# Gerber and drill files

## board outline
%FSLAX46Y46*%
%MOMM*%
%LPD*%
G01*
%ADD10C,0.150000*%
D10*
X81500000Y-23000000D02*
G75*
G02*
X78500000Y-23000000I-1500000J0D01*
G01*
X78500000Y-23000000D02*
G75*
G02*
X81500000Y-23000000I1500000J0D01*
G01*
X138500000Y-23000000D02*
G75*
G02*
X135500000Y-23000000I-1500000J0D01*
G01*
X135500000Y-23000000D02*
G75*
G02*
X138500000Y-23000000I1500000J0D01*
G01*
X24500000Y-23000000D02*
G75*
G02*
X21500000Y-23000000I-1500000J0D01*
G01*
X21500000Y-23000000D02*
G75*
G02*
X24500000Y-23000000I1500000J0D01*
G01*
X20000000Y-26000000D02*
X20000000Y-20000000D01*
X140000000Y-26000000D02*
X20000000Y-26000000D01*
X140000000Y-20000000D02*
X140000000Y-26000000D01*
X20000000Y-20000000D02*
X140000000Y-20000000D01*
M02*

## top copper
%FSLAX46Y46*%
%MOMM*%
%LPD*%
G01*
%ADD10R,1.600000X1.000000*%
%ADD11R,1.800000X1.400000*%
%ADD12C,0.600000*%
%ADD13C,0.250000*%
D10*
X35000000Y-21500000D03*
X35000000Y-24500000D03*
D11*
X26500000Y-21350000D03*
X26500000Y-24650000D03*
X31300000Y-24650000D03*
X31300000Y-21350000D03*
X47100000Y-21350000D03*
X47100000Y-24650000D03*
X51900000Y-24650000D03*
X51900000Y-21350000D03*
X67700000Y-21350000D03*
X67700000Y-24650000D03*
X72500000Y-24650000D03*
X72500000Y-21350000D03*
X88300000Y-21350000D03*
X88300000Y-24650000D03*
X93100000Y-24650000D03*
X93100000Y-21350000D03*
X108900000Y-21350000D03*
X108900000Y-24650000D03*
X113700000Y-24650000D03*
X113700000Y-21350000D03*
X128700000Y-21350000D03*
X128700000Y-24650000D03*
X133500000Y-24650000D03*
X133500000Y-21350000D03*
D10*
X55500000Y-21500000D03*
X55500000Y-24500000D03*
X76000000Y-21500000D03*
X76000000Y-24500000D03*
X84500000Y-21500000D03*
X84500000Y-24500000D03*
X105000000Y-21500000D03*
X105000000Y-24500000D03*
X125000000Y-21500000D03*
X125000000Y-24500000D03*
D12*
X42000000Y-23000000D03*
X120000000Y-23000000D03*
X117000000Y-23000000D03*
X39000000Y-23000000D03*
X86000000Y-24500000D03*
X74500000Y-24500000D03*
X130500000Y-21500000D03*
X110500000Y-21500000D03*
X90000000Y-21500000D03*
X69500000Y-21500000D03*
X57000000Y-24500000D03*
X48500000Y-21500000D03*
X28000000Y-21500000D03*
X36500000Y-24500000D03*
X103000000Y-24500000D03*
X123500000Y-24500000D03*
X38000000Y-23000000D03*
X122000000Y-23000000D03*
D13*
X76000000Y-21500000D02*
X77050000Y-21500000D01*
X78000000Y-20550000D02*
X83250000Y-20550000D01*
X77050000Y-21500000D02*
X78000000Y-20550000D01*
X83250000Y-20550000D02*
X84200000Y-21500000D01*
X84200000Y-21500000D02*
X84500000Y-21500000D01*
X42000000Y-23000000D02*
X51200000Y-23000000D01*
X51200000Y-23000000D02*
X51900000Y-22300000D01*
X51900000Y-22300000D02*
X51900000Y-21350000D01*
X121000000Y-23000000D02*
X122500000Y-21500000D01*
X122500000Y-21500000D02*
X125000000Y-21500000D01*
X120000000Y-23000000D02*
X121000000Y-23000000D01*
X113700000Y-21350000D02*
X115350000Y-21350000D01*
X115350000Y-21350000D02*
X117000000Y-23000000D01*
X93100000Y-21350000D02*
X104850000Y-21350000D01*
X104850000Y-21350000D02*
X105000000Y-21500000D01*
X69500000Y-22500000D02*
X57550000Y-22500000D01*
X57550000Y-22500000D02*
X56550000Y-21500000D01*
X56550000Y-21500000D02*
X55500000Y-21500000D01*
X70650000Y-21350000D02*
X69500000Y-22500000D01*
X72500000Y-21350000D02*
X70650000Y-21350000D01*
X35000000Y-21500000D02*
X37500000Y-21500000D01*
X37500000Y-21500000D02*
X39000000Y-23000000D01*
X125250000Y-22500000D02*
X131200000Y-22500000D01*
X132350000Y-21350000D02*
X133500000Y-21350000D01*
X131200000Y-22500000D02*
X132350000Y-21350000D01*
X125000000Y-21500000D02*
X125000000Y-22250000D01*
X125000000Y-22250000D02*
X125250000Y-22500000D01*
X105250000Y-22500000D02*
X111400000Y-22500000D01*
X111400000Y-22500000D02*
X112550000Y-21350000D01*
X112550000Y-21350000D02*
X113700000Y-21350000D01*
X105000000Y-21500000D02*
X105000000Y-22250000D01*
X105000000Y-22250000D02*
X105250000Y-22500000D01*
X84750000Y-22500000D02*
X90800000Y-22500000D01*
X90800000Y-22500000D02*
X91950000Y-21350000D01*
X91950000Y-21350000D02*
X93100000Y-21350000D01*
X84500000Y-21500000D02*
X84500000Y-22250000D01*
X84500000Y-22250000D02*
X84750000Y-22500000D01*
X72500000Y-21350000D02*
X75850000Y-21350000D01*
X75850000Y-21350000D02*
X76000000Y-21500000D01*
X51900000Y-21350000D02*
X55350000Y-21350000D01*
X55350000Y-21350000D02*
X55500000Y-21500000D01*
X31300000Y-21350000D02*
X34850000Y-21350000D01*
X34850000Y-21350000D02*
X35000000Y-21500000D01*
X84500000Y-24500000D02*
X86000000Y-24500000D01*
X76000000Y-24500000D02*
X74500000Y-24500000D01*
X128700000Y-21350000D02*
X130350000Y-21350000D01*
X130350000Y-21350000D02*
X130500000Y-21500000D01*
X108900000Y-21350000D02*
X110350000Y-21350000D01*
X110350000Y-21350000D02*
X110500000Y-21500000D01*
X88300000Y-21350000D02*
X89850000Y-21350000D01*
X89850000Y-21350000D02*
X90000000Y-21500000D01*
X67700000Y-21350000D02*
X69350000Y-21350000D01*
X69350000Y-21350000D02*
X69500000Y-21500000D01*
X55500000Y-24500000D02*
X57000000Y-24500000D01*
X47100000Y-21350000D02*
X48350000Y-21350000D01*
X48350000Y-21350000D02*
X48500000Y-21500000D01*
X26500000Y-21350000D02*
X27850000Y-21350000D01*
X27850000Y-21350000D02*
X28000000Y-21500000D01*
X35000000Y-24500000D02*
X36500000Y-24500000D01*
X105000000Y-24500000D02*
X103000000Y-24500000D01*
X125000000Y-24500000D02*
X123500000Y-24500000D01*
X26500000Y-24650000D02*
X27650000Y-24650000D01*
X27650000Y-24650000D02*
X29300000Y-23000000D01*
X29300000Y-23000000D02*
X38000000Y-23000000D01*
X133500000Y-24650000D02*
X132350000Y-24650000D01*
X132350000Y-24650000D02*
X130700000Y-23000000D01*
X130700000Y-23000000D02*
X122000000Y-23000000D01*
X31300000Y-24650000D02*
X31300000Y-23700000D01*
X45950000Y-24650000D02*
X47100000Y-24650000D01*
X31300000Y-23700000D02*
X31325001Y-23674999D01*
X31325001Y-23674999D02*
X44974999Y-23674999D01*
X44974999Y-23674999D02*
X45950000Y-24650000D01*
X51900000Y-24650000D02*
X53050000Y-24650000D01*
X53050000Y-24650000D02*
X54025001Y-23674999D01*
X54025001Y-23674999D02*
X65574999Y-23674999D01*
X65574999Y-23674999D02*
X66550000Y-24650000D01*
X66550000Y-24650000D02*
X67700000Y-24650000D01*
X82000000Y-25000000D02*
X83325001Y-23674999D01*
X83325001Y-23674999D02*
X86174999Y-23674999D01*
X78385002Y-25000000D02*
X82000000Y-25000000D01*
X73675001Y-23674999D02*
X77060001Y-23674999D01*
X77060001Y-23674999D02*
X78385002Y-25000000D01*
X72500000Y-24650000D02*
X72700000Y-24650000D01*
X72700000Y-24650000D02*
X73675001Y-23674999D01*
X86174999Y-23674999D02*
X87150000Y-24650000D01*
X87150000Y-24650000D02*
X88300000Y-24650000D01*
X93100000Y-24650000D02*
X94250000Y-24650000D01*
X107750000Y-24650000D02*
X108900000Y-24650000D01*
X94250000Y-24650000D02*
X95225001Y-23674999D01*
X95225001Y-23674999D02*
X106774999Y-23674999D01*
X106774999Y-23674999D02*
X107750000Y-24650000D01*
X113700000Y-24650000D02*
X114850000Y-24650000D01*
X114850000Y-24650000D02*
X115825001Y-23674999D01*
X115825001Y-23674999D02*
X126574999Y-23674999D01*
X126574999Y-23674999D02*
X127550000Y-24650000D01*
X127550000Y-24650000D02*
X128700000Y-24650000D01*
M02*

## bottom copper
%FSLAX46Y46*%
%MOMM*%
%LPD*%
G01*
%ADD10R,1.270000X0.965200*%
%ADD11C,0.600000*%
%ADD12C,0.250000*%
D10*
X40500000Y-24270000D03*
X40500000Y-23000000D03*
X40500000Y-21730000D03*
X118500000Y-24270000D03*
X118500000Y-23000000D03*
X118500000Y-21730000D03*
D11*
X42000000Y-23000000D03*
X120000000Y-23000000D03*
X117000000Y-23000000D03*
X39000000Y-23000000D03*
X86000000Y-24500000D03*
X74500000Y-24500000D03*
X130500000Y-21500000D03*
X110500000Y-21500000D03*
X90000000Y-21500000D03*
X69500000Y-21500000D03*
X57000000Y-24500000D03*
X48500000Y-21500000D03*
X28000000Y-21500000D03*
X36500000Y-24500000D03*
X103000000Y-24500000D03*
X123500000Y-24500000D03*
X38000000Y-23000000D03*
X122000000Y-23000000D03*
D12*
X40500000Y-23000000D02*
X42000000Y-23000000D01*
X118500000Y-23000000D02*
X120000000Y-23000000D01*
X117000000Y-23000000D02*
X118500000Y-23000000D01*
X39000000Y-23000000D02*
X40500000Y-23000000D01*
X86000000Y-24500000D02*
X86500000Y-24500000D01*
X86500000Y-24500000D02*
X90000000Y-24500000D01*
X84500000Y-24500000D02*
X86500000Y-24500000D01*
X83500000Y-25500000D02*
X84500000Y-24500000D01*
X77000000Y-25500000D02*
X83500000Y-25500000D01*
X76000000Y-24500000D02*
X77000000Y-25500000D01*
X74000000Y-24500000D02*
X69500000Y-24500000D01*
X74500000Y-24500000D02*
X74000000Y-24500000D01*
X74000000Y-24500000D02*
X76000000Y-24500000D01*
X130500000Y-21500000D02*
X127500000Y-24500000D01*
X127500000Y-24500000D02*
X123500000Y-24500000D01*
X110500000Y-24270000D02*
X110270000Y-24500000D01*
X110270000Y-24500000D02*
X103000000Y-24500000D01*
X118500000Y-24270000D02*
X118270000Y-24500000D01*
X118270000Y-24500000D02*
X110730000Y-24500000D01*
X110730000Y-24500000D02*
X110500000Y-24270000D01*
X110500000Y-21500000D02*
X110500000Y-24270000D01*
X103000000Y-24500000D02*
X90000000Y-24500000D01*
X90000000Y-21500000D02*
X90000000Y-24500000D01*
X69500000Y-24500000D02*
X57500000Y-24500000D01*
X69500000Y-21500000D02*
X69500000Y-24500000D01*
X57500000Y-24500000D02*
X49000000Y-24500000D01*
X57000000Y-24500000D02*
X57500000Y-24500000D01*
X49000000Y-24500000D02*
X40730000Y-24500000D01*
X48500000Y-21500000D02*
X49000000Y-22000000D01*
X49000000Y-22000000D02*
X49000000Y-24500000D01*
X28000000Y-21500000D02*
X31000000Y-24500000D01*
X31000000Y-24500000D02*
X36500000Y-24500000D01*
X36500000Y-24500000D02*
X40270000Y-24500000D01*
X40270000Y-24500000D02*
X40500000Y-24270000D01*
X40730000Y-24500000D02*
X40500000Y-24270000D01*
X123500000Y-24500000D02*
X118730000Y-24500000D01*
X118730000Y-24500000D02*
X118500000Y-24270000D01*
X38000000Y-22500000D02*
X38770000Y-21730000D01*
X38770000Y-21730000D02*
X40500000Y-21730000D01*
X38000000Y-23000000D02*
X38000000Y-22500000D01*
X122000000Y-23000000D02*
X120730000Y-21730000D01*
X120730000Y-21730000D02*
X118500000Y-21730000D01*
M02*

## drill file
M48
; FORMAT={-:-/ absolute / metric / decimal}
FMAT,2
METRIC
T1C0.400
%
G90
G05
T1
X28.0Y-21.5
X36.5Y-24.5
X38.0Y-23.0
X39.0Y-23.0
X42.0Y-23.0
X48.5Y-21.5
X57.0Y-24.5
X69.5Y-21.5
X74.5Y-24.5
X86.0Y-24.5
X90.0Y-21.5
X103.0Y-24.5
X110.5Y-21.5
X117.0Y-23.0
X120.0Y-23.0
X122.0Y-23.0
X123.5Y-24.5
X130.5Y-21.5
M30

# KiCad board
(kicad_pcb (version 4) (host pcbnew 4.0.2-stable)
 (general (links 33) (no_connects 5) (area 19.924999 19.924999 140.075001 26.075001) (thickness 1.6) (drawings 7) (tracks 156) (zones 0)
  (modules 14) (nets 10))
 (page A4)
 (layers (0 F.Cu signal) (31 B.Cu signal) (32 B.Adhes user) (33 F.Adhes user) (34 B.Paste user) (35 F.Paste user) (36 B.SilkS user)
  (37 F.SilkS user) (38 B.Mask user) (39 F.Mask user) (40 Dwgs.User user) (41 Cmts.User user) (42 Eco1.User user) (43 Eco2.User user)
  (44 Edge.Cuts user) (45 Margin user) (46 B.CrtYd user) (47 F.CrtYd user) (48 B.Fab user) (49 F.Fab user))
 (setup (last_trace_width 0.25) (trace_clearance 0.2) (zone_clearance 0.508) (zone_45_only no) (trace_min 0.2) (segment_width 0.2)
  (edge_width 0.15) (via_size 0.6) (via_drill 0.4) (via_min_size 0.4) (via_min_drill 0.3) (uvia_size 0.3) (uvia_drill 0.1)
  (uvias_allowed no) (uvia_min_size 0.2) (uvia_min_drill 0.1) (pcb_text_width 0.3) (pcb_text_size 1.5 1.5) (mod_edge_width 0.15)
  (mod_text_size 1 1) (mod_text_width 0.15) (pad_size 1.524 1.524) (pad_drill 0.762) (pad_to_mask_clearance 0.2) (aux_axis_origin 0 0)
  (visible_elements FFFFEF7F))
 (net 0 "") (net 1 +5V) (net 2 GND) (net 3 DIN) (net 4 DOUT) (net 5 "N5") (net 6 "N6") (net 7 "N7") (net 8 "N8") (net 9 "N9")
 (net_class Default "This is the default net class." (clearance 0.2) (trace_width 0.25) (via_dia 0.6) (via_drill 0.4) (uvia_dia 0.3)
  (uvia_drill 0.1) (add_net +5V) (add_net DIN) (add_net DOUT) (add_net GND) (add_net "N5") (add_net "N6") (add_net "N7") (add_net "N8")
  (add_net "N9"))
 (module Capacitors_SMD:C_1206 (layer F.Cu) (at 35 23 270)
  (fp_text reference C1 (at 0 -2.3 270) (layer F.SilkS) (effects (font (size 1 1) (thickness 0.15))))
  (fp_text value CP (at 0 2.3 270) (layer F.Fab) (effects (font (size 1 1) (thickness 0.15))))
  (pad 1 smd rect (at -1.5 0 270) (size 1 1.6) (layers F.Cu F.Paste F.Mask) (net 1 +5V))
  (pad 2 smd rect (at 1.5 0 270) (size 1 1.6) (layers F.Cu F.Paste F.Mask) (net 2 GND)))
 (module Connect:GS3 (layer B.Cu) (at 40.5 23)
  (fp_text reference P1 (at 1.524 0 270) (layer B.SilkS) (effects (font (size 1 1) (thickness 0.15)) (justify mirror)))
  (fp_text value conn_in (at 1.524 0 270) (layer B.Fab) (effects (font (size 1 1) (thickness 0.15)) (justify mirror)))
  (pad 1 smd rect (at 0 1.27) (size 1.27 0.9652) (layers B.Cu B.Paste B.Mask) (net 2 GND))
  (pad 2 smd rect (at 0 0) (size 1.27 0.9652) (layers B.Cu B.Paste B.Mask) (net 1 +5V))
  (pad 3 smd rect (at 0 -1.27) (size 1.27 0.9652) (layers B.Cu B.Paste B.Mask) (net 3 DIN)))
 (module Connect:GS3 (layer B.Cu) (at 118.5 23)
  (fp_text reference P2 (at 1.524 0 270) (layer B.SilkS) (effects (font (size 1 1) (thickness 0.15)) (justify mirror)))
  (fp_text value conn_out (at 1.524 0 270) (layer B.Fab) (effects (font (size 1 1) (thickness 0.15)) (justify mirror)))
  (pad 1 smd rect (at 0 1.27) (size 1.27 0.9652) (layers B.Cu B.Paste B.Mask) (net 2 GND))
  (pad 2 smd rect (at 0 0) (size 1.27 0.9652) (layers B.Cu B.Paste B.Mask) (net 1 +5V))
  (pad 3 smd rect (at 0 -1.27) (size 1.27 0.9652) (layers B.Cu B.Paste B.Mask) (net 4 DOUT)))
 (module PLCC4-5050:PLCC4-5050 (layer F.Cu) (at 28.9 23 90)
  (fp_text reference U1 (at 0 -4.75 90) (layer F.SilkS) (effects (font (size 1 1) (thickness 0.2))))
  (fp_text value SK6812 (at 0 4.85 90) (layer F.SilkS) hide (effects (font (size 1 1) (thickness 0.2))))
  (pad 1 smd rect (at 1.65 -2.4 90) (size 1.4 1.8) (layers F.Cu F.Paste F.Mask) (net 2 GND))
  (pad 2 smd rect (at -1.65 -2.4 90) (size 1.4 1.8) (layers F.Cu F.Paste F.Mask) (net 3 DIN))
  (pad 3 smd rect (at -1.65 2.4 90) (size 1.4 1.8) (layers F.Cu F.Paste F.Mask) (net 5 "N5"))
  (pad 4 smd rect (at 1.65 2.4 90) (size 1.4 1.8) (layers F.Cu F.Paste F.Mask) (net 1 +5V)))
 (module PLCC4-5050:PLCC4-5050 (layer F.Cu) (at 49.5 23 90)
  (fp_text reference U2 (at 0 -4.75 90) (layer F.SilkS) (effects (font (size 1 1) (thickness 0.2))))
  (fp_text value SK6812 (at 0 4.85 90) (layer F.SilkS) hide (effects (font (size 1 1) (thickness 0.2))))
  (pad 1 smd rect (at 1.65 -2.4 90) (size 1.4 1.8) (layers F.Cu F.Paste F.Mask) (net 2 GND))
  (pad 2 smd rect (at -1.65 -2.4 90) (size 1.4 1.8) (layers F.Cu F.Paste F.Mask) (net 5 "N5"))
  (pad 3 smd rect (at -1.65 2.4 90) (size 1.4 1.8) (layers F.Cu F.Paste F.Mask) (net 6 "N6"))
  (pad 4 smd rect (at 1.65 2.4 90) (size 1.4 1.8) (layers F.Cu F.Paste F.Mask) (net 1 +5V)))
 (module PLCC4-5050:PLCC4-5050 (layer F.Cu) (at 70.1 23 90)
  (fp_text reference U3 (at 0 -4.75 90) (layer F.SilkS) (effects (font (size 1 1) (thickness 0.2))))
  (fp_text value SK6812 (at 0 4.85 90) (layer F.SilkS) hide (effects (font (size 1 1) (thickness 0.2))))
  (pad 1 smd rect (at 1.65 -2.4 90) (size 1.4 1.8) (layers F.Cu F.Paste F.Mask) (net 2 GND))
  (pad 2 smd rect (at -1.65 -2.4 90) (size 1.4 1.8) (layers F.Cu F.Paste F.Mask) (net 6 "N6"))
  (pad 3 smd rect (at -1.65 2.4 90) (size 1.4 1.8) (layers F.Cu F.Paste F.Mask) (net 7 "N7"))
  (pad 4 smd rect (at 1.65 2.4 90) (size 1.4 1.8) (layers F.Cu F.Paste F.Mask) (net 1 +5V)))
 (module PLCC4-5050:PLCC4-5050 (layer F.Cu) (at 90.7 23 90) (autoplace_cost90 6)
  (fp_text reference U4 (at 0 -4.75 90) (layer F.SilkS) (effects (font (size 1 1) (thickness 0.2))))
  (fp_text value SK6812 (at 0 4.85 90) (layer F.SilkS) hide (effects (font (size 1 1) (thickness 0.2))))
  (pad 1 smd rect (at 1.65 -2.4 90) (size 1.4 1.8) (layers F.Cu F.Paste F.Mask) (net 2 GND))
  (pad 2 smd rect (at -1.65 -2.4 90) (size 1.4 1.8) (layers F.Cu F.Paste F.Mask) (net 7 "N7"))
  (pad 3 smd rect (at -1.65 2.4 90) (size 1.4 1.8) (layers F.Cu F.Paste F.Mask) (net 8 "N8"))
  (pad 4 smd rect (at 1.65 2.4 90) (size 1.4 1.8) (layers F.Cu F.Paste F.Mask) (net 1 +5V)))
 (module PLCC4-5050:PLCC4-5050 (layer F.Cu) (at 111.3 23 90)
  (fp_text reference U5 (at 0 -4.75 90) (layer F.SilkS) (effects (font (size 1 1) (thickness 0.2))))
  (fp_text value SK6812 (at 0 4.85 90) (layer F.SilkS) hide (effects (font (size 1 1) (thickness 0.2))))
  (pad 1 smd rect (at 1.65 -2.4 90) (size 1.4 1.8) (layers F.Cu F.Paste F.Mask) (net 2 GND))
  (pad 2 smd rect (at -1.65 -2.4 90) (size 1.4 1.8) (layers F.Cu F.Paste F.Mask) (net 8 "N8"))
  (pad 3 smd rect (at -1.65 2.4 90) (size 1.4 1.8) (layers F.Cu F.Paste F.Mask) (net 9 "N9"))
  (pad 4 smd rect (at 1.65 2.4 90) (size 1.4 1.8) (layers F.Cu F.Paste F.Mask) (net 1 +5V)))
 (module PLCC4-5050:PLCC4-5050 (layer F.Cu) (at 131.1 23 90)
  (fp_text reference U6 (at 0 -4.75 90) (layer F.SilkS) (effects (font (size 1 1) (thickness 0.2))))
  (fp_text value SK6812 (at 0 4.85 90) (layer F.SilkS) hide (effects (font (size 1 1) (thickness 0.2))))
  (pad 1 smd rect (at 1.65 -2.4 90) (size 1.4 1.8) (layers F.Cu F.Paste F.Mask) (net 2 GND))
  (pad 2 smd rect (at -1.65 -2.4 90) (size 1.4 1.8) (layers F.Cu F.Paste F.Mask) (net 9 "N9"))
  (pad 3 smd rect (at -1.65 2.4 90) (size 1.4 1.8) (layers F.Cu F.Paste F.Mask) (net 4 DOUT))
  (pad 4 smd rect (at 1.65 2.4 90) (size 1.4 1.8) (layers F.Cu F.Paste F.Mask) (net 1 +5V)))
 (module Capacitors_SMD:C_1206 (layer F.Cu) (at 55.5 23 270)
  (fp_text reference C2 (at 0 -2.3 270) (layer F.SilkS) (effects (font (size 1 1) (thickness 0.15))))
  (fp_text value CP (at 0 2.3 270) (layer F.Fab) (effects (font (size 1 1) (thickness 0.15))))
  (pad 1 smd rect (at -1.5 0 270) (size 1 1.6) (layers F.Cu F.Paste F.Mask) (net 1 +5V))
  (pad 2 smd rect (at 1.5 0 270) (size 1 1.6) (layers F.Cu F.Paste F.Mask) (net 2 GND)))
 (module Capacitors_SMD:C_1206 (layer F.Cu) (at 76 23 270)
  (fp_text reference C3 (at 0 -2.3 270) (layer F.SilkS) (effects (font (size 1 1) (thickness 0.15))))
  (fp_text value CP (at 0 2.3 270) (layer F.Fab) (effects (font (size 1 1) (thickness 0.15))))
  (pad 1 smd rect (at -1.5 0 270) (size 1 1.6) (layers F.Cu F.Paste F.Mask) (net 1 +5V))
  (pad 2 smd rect (at 1.5 0 270) (size 1 1.6) (layers F.Cu F.Paste F.Mask) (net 2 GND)))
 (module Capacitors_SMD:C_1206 (layer F.Cu) (at 84.5 23 270)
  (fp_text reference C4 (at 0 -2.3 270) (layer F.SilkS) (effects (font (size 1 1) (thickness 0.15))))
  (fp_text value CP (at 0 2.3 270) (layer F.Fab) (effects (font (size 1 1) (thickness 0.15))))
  (pad 1 smd rect (at -1.5 0 270) (size 1 1.6) (layers F.Cu F.Paste F.Mask) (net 1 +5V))
  (pad 2 smd rect (at 1.5 0 270) (size 1 1.6) (layers F.Cu F.Paste F.Mask) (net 2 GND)))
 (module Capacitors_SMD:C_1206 (layer F.Cu) (at 105 23 270)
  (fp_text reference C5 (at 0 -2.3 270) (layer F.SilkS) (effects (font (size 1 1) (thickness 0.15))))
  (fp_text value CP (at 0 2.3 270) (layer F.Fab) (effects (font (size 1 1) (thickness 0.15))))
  (pad 1 smd rect (at -1.5 0 270) (size 1 1.6) (layers F.Cu F.Paste F.Mask) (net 1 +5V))
  (pad 2 smd rect (at 1.5 0 270) (size 1 1.6) (layers F.Cu F.Paste F.Mask) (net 2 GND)))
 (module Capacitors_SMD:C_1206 (layer F.Cu) (at 125 23 270)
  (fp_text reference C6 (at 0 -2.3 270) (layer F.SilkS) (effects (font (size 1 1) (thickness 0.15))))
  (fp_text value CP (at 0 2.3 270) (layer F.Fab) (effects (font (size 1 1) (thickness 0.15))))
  (pad 1 smd rect (at -1.5 0 270) (size 1 1.6) (layers F.Cu F.Paste F.Mask) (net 1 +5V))
  (pad 2 smd rect (at 1.5 0 270) (size 1 1.6) (layers F.Cu F.Paste F.Mask) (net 2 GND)))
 (gr_circle (center 80 23) (end 80 24.5) (layer Edge.Cuts) (width 0.15))
 (gr_circle (center 137 23) (end 137 24.5) (layer Edge.Cuts) (width 0.15))
 (gr_circle (center 23 23) (end 23 24.5) (layer Edge.Cuts) (width 0.15))
 (gr_line (start 20 26) (end 20 20) (layer Edge.Cuts) (width 0.15))
 (gr_line (start 140 26) (end 20 26) (layer Edge.Cuts) (width 0.15))
 (gr_line (start 140 20) (end 140 26) (layer Edge.Cuts) (width 0.15))
 (gr_line (start 20 20) (end 140 20) (layer Edge.Cuts) (width 0.15))
 (segment (start 76 21.5) (end 77.05 21.5) (width 0.25) (layer F.Cu) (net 1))
 (segment (start 78 20.55) (end 83.25 20.55) (width 0.25) (layer F.Cu) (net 1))
 (segment (start 77.05 21.5) (end 78 20.55) (width 0.25) (layer F.Cu) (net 1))
 (segment (start 83.25 20.55) (end 84.2 21.5) (width 0.25) (layer F.Cu) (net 1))
 (segment (start 84.2 21.5) (end 84.5 21.5) (width 0.25) (layer F.Cu) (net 1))
 (segment (start 42 23) (end 51.2 23) (width 0.25) (layer F.Cu) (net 1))
 (segment (start 51.2 23) (end 51.9 22.3) (width 0.25) (layer F.Cu) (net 1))
 (segment (start 51.9 22.3) (end 51.9 21.35) (width 0.25) (layer F.Cu) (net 1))
 (segment (start 40.5 23) (end 42 23) (width 0.25) (layer B.Cu) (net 1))
 (via (at 42 23) (size 0.6) (drill 0.4) (layers F.Cu B.Cu) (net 1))
 (segment (start 121 23) (end 122.5 21.5) (width 0.25) (layer F.Cu) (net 1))
 (segment (start 122.5 21.5) (end 125 21.5) (width 0.25) (layer F.Cu) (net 1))
 (segment (start 120 23) (end 121 23) (width 0.25) (layer F.Cu) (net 1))
 (segment (start 118.5 23) (end 120 23) (width 0.25) (layer B.Cu) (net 1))
 (via (at 120 23) (size 0.6) (drill 0.4) (layers F.Cu B.Cu) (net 1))
 (segment (start 117 23) (end 118.5 23) (width 0.25) (layer B.Cu) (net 1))
 (segment (start 113.7 21.35) (end 115.35 21.35) (width 0.25) (layer F.Cu) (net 1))
 (segment (start 115.35 21.35) (end 117 23) (width 0.25) (layer F.Cu) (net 1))
 (via (at 117 23) (size 0.6) (drill 0.4) (layers F.Cu B.Cu) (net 1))
 (segment (start 93.1 21.35) (end 104.85 21.35) (width 0.25) (layer F.Cu) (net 1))
 (segment (start 104.85 21.35) (end 105 21.5) (width 0.25) (layer F.Cu) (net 1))
 (segment (start 69.5 22.5) (end 57.55 22.5) (width 0.25) (layer F.Cu) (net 1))
 (segment (start 57.55 22.5) (end 56.55 21.5) (width 0.25) (layer F.Cu) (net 1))
 (segment (start 56.55 21.5) (end 55.5 21.5) (width 0.25) (layer F.Cu) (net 1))
 (segment (start 70.65 21.35) (end 69.5 22.5) (width 0.25) (layer F.Cu) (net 1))
 (segment (start 72.5 21.35) (end 70.65 21.35) (width 0.25) (layer F.Cu) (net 1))
 (segment (start 39 23) (end 40.5 23) (width 0.25) (layer B.Cu) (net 1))
 (segment (start 35 21.5) (end 37.5 21.5) (width 0.25) (layer F.Cu) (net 1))
 (segment (start 37.5 21.5) (end 39 23) (width 0.25) (layer F.Cu) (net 1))
 (via (at 39 23) (size 0.6) (drill 0.4) (layers F.Cu B.Cu) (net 1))
 (segment (start 125.25 22.5) (end 131.2 22.5) (width 0.25) (layer F.Cu) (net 1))
 (segment (start 132.35 21.35) (end 133.5 21.35) (width 0.25) (layer F.Cu) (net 1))
 (segment (start 131.2 22.5) (end 132.35 21.35) (width 0.25) (layer F.Cu) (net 1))
 (segment (start 125 21.5) (end 125 22.25) (width 0.25) (layer F.Cu) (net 1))
 (segment (start 125 22.25) (end 125.25 22.5) (width 0.25) (layer F.Cu) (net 1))
 (segment (start 105.25 22.5) (end 111.4 22.5) (width 0.25) (layer F.Cu) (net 1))
 (segment (start 111.4 22.5) (end 112.55 21.35) (width 0.25) (layer F.Cu) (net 1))
 (segment (start 112.55 21.35) (end 113.7 21.35) (width 0.25) (layer F.Cu) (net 1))
 (segment (start 105 21.5) (end 105 22.25) (width 0.25) (layer F.Cu) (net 1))
 (segment (start 105 22.25) (end 105.25 22.5) (width 0.25) (layer F.Cu) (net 1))
 (segment (start 84.75 22.5) (end 90.8 22.5) (width 0.25) (layer F.Cu) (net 1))
 (segment (start 90.8 22.5) (end 91.95 21.35) (width 0.25) (layer F.Cu) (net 1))
 (segment (start 91.95 21.35) (end 93.1 21.35) (width 0.25) (layer F.Cu) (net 1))
 (segment (start 84.5 21.5) (end 84.5 22.25) (width 0.25) (layer F.Cu) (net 1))
 (segment (start 84.5 22.25) (end 84.75 22.5) (width 0.25) (layer F.Cu) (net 1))
 (segment (start 72.5 21.35) (end 75.85 21.35) (width 0.25) (layer F.Cu) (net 1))
 (segment (start 75.85 21.35) (end 76 21.5) (width 0.25) (layer F.Cu) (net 1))
 (segment (start 51.9 21.35) (end 55.35 21.35) (width 0.25) (layer F.Cu) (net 1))
 (segment (start 55.35 21.35) (end 55.5 21.5) (width 0.25) (layer F.Cu) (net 1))
 (segment (start 31.3 21.35) (end 34.85 21.35) (width 0.25) (layer F.Cu) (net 1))
 (segment (start 34.85 21.35) (end 35 21.5) (width 0.25) (layer F.Cu) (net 1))
 (segment (start 86 24.5) (end 86.5 24.5) (width 0.25) (layer B.Cu) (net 2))
 (segment (start 86.5 24.5) (end 90 24.5) (width 0.25) (layer B.Cu) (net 2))
 (segment (start 84.5 24.5) (end 86.5 24.5) (width 0.25) (layer B.Cu) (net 2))
 (segment (start 83.5 25.5) (end 84.5 24.5) (width 0.25) (layer B.Cu) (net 2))
 (segment (start 77 25.5) (end 83.5 25.5) (width 0.25) (layer B.Cu) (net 2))
 (segment (start 76 24.5) (end 77 25.5) (width 0.25) (layer B.Cu) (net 2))
 (segment (start 74 24.5) (end 69.5 24.5) (width 0.25) (layer B.Cu) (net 2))
 (segment (start 74.5 24.5) (end 74 24.5) (width 0.25) (layer B.Cu) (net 2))
 (segment (start 74 24.5) (end 76 24.5) (width 0.25) (layer B.Cu) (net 2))
 (segment (start 84.5 24.5) (end 86 24.5) (width 0.25) (layer F.Cu) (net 2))
 (via (at 86 24.5) (size 0.6) (drill 0.4) (layers F.Cu B.Cu) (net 2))
 (segment (start 76 24.5) (end 74.5 24.5) (width 0.25) (layer F.Cu) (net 2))
 (via (at 74.5 24.5) (size 0.6) (drill 0.4) (layers F.Cu B.Cu) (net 2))
 (segment (start 130.5 21.5) (end 127.5 24.5) (width 0.25) (layer B.Cu) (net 2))
 (segment (start 127.5 24.5) (end 123.5 24.5) (width 0.25) (layer B.Cu) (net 2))
 (segment (start 128.7 21.35) (end 130.35 21.35) (width 0.25) (layer F.Cu) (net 2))
 (segment (start 130.35 21.35) (end 130.5 21.5) (width 0.25) (layer F.Cu) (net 2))
 (via (at 130.5 21.5) (size 0.6) (drill 0.4) (layers F.Cu B.Cu) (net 2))
 (segment (start 110.5 24.27) (end 110.27 24.5) (width 0.25) (layer B.Cu) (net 2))
 (segment (start 110.27 24.5) (end 103 24.5) (width 0.25) (layer B.Cu) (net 2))
 (segment (start 118.5 24.27) (end 118.27 24.5) (width 0.25) (layer B.Cu) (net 2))
 (segment (start 118.27 24.5) (end 110.73 24.5) (width 0.25) (layer B.Cu) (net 2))
 (segment (start 110.73 24.5) (end 110.5 24.27) (width 0.25) (layer B.Cu) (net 2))
 (segment (start 110.5 21.5) (end 110.5 24.27) (width 0.25) (layer B.Cu) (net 2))
 (segment (start 108.9 21.35) (end 110.35 21.35) (width 0.25) (layer F.Cu) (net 2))
 (segment (start 110.35 21.35) (end 110.5 21.5) (width 0.25) (layer F.Cu) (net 2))
 (via (at 110.5 21.5) (size 0.6) (drill 0.4) (layers F.Cu B.Cu) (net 2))
 (segment (start 103 24.5) (end 90 24.5) (width 0.25) (layer B.Cu) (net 2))
 (segment (start 90 21.5) (end 90 24.5) (width 0.25) (layer B.Cu) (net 2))
 (segment (start 88.3 21.35) (end 89.85 21.35) (width 0.25) (layer F.Cu) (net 2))
 (segment (start 89.85 21.35) (end 90 21.5) (width 0.25) (layer F.Cu) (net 2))
 (via (at 90 21.5) (size 0.6) (drill 0.4) (layers F.Cu B.Cu) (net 2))
 (segment (start 69.5 24.5) (end 57.5 24.5) (width 0.25) (layer B.Cu) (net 2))
 (segment (start 69.5 21.5) (end 69.5 24.5) (width 0.25) (layer B.Cu) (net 2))
 (segment (start 67.7 21.35) (end 69.35 21.35) (width 0.25) (layer F.Cu) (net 2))
 (segment (start 69.35 21.35) (end 69.5 21.5) (width 0.25) (layer F.Cu) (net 2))
 (via (at 69.5 21.5) (size 0.6) (drill 0.4) (layers F.Cu B.Cu) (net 2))
 (segment (start 57.5 24.5) (end 49 24.5) (width 0.25) (layer B.Cu) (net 2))
 (segment (start 57 24.5) (end 57.5 24.5) (width 0.25) (layer B.Cu) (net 2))
 (segment (start 55.5 24.5) (end 57 24.5) (width 0.25) (layer F.Cu) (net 2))
 (via (at 57 24.5) (size 0.6) (drill 0.4) (layers F.Cu B.Cu) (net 2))
 (segment (start 49 24.5) (end 40.73 24.5) (width 0.25) (layer B.Cu) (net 2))
 (segment (start 48.5 21.5) (end 49 22) (width 0.25) (layer B.Cu) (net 2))
 (segment (start 49 22) (end 49 24.5) (width 0.25) (layer B.Cu) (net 2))
 (segment (start 47.1 21.35) (end 48.35 21.35) (width 0.25) (layer F.Cu) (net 2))
 (via (at 48.5 21.5) (size 0.6) (drill 0.4) (layers F.Cu B.Cu) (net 2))
 (segment (start 48.35 21.35) (end 48.5 21.5) (width 0.25) (layer F.Cu) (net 2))
 (segment (start 28 21.5) (end 31 24.5) (width 0.25) (layer B.Cu) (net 2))
 (segment (start 31 24.5) (end 36.5 24.5) (width 0.25) (layer B.Cu) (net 2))
 (segment (start 26.5 21.35) (end 27.85 21.35) (width 0.25) (layer F.Cu) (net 2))
 (segment (start 27.85 21.35) (end 28 21.5) (width 0.25) (layer F.Cu) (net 2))
 (via (at 28 21.5) (size 0.6) (drill 0.4) (layers F.Cu B.Cu) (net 2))
 (segment (start 36.5 24.5) (end 40.27 24.5) (width 0.25) (layer B.Cu) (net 2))
 (segment (start 40.27 24.5) (end 40.5 24.27) (width 0.25) (layer B.Cu) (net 2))
 (segment (start 35 24.5) (end 36.5 24.5) (width 0.25) (layer F.Cu) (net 2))
 (via (at 36.5 24.5) (size 0.6) (drill 0.4) (layers F.Cu B.Cu) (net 2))
 (segment (start 40.73 24.5) (end 40.5 24.27) (width 0.25) (layer B.Cu) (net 2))
 (segment (start 105 24.5) (end 103 24.5) (width 0.25) (layer F.Cu) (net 2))
 (via (at 103 24.5) (size 0.6) (drill 0.4) (layers F.Cu B.Cu) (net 2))
 (segment (start 123.5 24.5) (end 118.73 24.5) (width 0.25) (layer B.Cu) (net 2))
 (segment (start 118.73 24.5) (end 118.5 24.27) (width 0.25) (layer B.Cu) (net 2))
 (segment (start 125 24.5) (end 123.5 24.5) (width 0.25) (layer F.Cu) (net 2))
 (via (at 123.5 24.5) (size 0.6) (drill 0.4) (layers F.Cu B.Cu) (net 2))
 (segment (start 38 22.5) (end 38.77 21.73) (width 0.25) (layer B.Cu) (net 3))
 (segment (start 38.77 21.73) (end 40.5 21.73) (width 0.25) (layer B.Cu) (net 3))
 (segment (start 38 23) (end 38 22.5) (width 0.25) (layer B.Cu) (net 3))
 (segment (start 26.5 24.65) (end 27.65 24.65) (width 0.25) (layer F.Cu) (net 3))
 (segment (start 27.65 24.65) (end 29.3 23) (width 0.25) (layer F.Cu) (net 3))
 (segment (start 29.3 23) (end 38 23) (width 0.25) (layer F.Cu) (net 3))
 (via (at 38 23) (size 0.6) (drill 0.4) (layers F.Cu B.Cu) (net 3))
 (segment (start 122 23) (end 120.73 21.73) (width 0.25) (layer B.Cu) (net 4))
 (segment (start 120.73 21.73) (end 118.5 21.73) (width 0.25) (layer B.Cu) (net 4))
 (segment (start 133.5 24.65) (end 132.35 24.65) (width 0.25) (layer F.Cu) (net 4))
 (segment (start 132.35 24.65) (end 130.7 23) (width 0.25) (layer F.Cu) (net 4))
 (segment (start 130.7 23) (end 122 23) (width 0.25) (layer F.Cu) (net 4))
 (via (at 122 23) (size 0.6) (drill 0.4) (layers F.Cu B.Cu) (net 4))
 (segment (start 31.3 24.65) (end 31.3 23.7) (width 0.25) (layer F.Cu) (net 5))
 (segment (start 45.95 24.65) (end 47.1 24.65) (width 0.25) (layer F.Cu) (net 5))
 (segment (start 31.3 23.7) (end 31.325001 23.674999) (width 0.25) (layer F.Cu) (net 5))
 (segment (start 31.325001 23.674999) (end 44.974999 23.674999) (width 0.25) (layer F.Cu) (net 5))
 (segment (start 44.974999 23.674999) (end 45.95 24.65) (width 0.25) (layer F.Cu) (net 5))
 (segment (start 51.9 24.65) (end 53.05 24.65) (width 0.25) (layer F.Cu) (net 6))
 (segment (start 53.05 24.65) (end 54.025001 23.674999) (width 0.25) (layer F.Cu) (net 6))
 (segment (start 54.025001 23.674999) (end 65.574999 23.674999) (width 0.25) (layer F.Cu) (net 6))
 (segment (start 65.574999 23.674999) (end 66.55 24.65) (width 0.25) (layer F.Cu) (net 6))
 (segment (start 66.55 24.65) (end 67.7 24.65) (width 0.25) (layer F.Cu) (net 6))
 (segment (start 82 25) (end 83.325001 23.674999) (width 0.25) (layer F.Cu) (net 7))
 (segment (start 83.325001 23.674999) (end 86.174999 23.674999) (width 0.25) (layer F.Cu) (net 7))
 (segment (start 78.385002 25) (end 82 25) (width 0.25) (layer F.Cu) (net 7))
 (segment (start 73.675001 23.674999) (end 77.060001 23.674999) (width 0.25) (layer F.Cu) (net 7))
 (segment (start 77.060001 23.674999) (end 78.385002 25) (width 0.25) (layer F.Cu) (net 7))
 (segment (start 72.5 24.65) (end 72.7 24.65) (width 0.25) (layer F.Cu) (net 7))
 (segment (start 72.7 24.65) (end 73.675001 23.674999) (width 0.25) (layer F.Cu) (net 7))
 (segment (start 86.174999 23.674999) (end 87.15 24.65) (width 0.25) (layer F.Cu) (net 7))
 (segment (start 87.15 24.65) (end 88.3 24.65) (width 0.25) (layer F.Cu) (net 7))
 (segment (start 93.1 24.65) (end 94.25 24.65) (width 0.25) (layer F.Cu) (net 8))
 (segment (start 107.75 24.65) (end 108.9 24.65) (width 0.25) (layer F.Cu) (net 8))
 (segment (start 94.25 24.65) (end 95.225001 23.674999) (width 0.25) (layer F.Cu) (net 8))
 (segment (start 95.225001 23.674999) (end 106.774999 23.674999) (width 0.25) (layer F.Cu) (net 8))
 (segment (start 106.774999 23.674999) (end 107.75 24.65) (width 0.25) (layer F.Cu) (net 8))
 (segment (start 113.7 24.65) (end 114.85 24.65) (width 0.25) (layer F.Cu) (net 9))
 (segment (start 114.85 24.65) (end 115.825001 23.674999) (width 0.25) (layer F.Cu) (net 9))
 (segment (start 115.825001 23.674999) (end 126.574999 23.674999) (width 0.25) (layer F.Cu) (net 9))
 (segment (start 126.574999 23.674999) (end 127.55 24.65) (width 0.25) (layer F.Cu) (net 9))
 (segment (start 127.55 24.65) (end 128.7 24.65) (width 0.25) (layer F.Cu) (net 9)))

